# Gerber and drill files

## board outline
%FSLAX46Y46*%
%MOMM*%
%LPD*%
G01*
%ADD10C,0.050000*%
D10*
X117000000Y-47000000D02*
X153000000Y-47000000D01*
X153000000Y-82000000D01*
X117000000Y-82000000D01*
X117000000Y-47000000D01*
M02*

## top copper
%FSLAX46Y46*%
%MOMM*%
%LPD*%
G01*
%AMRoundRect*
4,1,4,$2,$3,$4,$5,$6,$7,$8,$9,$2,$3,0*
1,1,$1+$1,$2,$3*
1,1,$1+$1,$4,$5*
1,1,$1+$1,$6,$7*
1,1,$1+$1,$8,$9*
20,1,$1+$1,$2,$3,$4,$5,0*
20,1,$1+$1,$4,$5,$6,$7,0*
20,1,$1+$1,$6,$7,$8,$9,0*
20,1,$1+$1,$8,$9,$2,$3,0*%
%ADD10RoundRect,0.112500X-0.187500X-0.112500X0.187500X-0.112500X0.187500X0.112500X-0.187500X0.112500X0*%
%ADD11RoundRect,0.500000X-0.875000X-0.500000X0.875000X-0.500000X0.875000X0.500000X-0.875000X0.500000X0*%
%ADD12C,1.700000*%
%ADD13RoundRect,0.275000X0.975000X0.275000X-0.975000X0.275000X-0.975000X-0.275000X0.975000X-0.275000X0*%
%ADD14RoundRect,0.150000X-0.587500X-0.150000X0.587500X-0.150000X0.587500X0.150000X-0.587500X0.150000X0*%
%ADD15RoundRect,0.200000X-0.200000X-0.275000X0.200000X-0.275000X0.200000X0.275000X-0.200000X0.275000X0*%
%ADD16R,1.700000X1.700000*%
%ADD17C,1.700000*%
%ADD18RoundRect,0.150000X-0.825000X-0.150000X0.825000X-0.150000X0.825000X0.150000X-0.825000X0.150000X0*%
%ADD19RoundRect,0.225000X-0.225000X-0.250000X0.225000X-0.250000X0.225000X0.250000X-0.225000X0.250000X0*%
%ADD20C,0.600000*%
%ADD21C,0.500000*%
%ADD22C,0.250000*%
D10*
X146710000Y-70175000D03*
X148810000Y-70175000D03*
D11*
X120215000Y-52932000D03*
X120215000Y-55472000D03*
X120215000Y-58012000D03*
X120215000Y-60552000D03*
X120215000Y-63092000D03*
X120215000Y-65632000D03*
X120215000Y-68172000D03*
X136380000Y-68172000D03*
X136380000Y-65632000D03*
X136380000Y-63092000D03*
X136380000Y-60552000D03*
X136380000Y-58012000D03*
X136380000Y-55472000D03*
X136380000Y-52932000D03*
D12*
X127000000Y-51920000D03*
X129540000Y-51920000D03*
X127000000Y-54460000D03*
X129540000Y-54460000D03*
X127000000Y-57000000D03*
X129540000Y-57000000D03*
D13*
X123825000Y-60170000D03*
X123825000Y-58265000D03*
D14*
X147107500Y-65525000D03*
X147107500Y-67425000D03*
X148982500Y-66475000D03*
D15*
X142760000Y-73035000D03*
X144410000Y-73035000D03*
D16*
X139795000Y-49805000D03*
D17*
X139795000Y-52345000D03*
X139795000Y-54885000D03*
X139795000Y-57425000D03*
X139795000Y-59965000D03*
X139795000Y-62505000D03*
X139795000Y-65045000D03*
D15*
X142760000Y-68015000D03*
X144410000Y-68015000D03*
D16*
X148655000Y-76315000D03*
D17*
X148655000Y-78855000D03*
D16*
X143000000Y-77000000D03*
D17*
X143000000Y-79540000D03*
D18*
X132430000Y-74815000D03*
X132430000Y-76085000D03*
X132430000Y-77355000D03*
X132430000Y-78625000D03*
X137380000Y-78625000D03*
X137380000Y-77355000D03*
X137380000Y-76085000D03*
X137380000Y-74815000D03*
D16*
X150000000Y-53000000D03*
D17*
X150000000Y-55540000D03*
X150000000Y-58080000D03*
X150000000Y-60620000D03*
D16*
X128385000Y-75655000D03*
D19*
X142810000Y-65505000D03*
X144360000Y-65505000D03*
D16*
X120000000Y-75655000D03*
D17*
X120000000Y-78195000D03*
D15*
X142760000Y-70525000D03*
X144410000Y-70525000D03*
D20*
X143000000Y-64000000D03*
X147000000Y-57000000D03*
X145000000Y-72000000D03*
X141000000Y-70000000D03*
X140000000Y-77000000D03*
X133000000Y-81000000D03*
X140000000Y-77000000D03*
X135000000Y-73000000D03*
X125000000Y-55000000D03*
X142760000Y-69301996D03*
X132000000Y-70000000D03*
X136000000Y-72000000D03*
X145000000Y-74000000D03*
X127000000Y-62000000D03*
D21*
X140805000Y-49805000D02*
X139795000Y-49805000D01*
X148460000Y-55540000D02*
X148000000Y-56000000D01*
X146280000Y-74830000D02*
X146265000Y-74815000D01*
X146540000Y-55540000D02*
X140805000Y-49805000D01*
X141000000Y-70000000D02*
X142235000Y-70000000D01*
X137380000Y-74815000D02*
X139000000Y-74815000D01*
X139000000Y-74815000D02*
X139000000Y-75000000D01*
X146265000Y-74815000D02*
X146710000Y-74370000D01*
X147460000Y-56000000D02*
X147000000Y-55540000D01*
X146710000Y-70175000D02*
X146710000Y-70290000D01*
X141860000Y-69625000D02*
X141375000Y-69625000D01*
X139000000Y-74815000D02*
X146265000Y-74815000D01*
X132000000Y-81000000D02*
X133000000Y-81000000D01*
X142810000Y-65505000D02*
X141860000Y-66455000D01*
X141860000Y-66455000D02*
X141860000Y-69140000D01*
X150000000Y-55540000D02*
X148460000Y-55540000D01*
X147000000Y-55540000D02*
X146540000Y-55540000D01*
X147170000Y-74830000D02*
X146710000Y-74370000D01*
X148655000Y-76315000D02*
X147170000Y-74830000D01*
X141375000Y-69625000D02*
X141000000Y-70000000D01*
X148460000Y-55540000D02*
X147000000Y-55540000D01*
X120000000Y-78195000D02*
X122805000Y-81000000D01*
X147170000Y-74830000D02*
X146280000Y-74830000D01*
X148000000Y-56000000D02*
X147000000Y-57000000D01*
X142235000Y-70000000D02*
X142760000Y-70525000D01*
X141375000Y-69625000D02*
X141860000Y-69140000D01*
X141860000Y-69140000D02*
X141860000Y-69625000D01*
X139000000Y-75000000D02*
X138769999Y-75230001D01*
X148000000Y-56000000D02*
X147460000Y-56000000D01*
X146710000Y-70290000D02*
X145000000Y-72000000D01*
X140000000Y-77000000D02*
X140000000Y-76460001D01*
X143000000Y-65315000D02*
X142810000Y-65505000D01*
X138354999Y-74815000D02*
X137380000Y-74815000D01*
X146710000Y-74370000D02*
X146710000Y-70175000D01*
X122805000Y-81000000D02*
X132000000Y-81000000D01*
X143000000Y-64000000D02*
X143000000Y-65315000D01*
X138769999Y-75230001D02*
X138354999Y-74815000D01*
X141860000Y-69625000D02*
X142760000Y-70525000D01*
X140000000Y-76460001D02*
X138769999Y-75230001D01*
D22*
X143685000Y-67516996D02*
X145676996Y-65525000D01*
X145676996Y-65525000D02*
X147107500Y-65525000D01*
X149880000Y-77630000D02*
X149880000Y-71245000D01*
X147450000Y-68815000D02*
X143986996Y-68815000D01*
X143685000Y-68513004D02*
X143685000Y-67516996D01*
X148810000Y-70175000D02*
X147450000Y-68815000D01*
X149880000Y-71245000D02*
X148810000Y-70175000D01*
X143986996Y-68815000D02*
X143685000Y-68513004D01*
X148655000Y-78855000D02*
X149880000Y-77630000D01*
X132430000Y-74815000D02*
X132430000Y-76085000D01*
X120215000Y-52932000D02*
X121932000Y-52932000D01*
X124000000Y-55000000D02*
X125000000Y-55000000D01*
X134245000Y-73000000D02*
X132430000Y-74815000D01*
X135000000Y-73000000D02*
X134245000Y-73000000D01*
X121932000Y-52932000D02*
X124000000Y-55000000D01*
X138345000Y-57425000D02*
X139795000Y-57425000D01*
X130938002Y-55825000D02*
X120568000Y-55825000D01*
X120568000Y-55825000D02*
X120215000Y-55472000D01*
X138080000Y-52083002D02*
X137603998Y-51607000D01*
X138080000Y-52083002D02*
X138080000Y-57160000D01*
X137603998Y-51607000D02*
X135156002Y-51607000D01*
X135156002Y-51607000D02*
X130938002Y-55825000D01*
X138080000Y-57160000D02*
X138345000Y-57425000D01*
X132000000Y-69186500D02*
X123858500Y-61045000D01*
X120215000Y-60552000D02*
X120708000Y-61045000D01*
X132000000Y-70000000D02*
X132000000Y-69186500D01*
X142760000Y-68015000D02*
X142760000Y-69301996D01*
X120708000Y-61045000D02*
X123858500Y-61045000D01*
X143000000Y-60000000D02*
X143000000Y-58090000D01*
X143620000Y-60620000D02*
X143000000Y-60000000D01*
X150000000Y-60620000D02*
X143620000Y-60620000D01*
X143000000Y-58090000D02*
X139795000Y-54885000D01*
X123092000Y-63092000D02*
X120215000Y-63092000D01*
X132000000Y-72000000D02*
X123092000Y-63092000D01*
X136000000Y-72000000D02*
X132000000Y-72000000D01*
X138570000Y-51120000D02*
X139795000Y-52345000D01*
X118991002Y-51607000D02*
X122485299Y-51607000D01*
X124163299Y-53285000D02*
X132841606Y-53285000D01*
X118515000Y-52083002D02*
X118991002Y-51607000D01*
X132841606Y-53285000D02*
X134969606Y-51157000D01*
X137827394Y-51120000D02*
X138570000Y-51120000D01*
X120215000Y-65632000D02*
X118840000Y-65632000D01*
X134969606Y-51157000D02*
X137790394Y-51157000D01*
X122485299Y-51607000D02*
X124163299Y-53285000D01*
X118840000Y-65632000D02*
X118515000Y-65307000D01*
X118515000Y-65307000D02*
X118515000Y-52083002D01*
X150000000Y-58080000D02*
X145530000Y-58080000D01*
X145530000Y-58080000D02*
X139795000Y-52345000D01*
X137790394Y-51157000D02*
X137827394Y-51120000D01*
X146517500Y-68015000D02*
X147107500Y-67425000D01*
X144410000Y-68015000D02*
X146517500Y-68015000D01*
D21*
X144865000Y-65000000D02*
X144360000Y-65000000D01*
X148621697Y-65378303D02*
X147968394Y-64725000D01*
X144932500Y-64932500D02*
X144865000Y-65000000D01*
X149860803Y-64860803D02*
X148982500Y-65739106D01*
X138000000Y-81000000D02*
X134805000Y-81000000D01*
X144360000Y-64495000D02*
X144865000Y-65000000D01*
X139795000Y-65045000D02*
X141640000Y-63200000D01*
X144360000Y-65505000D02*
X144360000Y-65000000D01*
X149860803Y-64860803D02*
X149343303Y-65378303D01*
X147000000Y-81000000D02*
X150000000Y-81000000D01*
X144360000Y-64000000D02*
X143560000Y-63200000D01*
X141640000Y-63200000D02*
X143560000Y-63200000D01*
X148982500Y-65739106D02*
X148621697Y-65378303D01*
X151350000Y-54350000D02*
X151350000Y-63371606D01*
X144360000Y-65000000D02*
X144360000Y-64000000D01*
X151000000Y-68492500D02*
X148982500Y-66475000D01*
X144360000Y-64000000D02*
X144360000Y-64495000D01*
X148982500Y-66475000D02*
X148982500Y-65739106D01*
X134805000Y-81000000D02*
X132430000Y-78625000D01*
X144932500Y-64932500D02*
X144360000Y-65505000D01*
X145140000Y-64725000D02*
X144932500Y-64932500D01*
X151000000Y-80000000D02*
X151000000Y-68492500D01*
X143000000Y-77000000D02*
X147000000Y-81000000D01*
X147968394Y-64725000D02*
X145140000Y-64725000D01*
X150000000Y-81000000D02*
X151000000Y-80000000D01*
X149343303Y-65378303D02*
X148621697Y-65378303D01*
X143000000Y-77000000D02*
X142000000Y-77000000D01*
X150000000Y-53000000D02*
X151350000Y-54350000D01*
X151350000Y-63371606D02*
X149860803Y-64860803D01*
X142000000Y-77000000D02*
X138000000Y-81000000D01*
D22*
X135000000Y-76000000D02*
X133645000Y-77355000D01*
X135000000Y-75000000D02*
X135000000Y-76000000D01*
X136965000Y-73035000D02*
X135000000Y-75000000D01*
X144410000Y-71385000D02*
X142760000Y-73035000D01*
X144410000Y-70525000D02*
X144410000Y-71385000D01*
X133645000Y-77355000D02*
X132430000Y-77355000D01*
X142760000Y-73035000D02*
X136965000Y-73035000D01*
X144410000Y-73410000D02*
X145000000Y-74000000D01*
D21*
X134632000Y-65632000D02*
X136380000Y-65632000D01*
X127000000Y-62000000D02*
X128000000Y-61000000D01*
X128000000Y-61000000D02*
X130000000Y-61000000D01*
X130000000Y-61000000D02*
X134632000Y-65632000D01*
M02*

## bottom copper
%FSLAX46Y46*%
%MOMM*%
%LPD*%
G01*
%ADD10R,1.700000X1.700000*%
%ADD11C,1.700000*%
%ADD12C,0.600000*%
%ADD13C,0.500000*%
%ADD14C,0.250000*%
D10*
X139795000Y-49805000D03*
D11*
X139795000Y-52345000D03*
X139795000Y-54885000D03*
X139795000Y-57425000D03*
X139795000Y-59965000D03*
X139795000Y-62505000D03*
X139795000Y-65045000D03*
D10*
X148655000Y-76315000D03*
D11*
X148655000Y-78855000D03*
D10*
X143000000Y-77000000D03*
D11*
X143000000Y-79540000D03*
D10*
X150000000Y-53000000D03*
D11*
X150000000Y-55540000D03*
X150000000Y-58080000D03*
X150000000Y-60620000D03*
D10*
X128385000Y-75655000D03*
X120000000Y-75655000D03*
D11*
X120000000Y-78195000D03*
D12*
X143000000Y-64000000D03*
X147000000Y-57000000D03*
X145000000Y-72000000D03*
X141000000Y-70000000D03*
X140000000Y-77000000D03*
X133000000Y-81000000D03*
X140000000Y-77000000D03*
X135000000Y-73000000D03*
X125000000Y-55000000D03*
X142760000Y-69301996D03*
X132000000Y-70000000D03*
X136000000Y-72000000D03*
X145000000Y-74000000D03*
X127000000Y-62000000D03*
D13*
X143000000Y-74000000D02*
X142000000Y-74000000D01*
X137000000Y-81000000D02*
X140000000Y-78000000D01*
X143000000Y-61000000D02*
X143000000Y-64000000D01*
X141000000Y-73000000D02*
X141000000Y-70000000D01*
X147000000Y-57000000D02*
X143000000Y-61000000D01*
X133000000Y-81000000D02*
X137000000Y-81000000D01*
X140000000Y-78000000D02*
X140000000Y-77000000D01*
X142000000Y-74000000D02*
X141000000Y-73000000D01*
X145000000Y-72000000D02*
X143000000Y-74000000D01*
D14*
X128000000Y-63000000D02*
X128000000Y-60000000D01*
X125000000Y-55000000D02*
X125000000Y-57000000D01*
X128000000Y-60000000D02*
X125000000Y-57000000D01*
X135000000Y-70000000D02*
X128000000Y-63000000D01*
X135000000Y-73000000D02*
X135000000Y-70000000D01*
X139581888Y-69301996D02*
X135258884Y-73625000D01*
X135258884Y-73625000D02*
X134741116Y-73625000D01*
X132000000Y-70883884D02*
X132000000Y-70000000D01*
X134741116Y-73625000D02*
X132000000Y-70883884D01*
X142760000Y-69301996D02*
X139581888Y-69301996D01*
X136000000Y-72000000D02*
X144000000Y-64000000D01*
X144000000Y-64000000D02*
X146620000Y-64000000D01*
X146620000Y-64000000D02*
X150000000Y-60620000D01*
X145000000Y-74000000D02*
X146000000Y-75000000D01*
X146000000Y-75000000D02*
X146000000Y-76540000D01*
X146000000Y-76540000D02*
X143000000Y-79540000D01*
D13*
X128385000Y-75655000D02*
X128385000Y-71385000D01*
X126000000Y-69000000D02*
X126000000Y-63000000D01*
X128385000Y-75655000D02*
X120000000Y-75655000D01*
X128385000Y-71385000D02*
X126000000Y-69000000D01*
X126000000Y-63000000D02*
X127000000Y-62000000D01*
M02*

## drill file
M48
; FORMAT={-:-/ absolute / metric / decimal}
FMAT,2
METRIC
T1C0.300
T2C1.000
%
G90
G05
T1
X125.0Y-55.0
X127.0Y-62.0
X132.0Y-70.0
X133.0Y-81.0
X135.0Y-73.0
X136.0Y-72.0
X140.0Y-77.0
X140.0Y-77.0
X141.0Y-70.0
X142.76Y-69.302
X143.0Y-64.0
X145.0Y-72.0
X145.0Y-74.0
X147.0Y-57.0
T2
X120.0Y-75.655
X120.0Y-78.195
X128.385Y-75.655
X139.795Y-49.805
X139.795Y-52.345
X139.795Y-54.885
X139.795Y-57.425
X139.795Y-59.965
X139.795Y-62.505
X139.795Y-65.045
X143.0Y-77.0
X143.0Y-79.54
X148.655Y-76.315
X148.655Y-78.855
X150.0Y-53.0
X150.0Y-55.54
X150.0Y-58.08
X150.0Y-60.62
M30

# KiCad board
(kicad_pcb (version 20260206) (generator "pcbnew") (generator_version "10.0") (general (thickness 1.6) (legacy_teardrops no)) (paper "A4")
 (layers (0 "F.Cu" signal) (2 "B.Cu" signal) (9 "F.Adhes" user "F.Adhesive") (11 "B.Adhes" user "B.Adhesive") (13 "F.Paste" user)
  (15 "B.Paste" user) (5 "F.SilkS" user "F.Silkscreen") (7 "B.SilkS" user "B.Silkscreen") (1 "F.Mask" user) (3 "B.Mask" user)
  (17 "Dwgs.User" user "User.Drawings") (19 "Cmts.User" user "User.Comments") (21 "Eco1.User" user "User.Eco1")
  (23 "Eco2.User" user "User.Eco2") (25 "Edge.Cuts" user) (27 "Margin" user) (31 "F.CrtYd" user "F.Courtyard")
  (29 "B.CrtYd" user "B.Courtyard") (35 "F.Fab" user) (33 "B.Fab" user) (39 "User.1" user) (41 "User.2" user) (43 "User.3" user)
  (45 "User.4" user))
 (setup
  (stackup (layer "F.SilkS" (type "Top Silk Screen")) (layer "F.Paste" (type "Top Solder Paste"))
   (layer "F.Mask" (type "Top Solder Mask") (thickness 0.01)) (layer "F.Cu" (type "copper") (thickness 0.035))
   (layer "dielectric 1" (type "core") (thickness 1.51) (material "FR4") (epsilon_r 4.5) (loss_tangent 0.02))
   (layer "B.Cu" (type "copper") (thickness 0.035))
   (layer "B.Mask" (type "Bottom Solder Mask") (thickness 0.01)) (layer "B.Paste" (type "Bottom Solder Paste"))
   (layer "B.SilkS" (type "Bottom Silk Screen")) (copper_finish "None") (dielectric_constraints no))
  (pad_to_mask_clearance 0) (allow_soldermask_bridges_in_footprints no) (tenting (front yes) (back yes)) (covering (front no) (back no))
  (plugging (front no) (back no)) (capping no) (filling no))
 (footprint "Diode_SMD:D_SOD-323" (layer "F.Cu") (at 147.76 70.175)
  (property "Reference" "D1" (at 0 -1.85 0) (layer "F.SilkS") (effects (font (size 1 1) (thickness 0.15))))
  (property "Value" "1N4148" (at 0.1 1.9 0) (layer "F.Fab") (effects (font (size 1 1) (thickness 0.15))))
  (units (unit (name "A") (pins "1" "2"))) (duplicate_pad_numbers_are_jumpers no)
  (pad "1" smd roundrect (at -1.05 0) (size 0.6 0.45) (layers "F.Cu" "F.Mask" "F.Paste") (roundrect_rratio 0.25) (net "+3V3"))
  (pad "2" smd roundrect (at 1.05 0) (size 0.6 0.45) (layers "F.Cu" "F.Mask" "F.Paste") (roundrect_rratio 0.25) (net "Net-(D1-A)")))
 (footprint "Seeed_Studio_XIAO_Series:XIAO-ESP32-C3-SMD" (layer "F.Cu") (at 119.38 71.052)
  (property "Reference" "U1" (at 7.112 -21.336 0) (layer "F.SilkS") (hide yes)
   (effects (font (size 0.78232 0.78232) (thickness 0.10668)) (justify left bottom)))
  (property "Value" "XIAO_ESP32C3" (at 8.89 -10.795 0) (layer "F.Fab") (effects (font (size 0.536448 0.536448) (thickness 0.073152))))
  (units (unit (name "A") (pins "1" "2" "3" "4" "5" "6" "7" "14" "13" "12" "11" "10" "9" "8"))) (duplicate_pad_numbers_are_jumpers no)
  (pad "1" smd roundrect (at 0.835 -18.12) (size 2.75 2) (layers "F.Cu" "F.Mask" "F.Paste") (roundrect_rratio 0.25) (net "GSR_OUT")
   (solder_mask_margin 0.0508) (thermal_bridge_angle 45))
  (pad "2" smd roundrect (at 0.835 -15.58) (size 2.75 2) (layers "F.Cu" "F.Mask" "F.Paste") (roundrect_rratio 0.25) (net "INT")
   (solder_mask_margin 0.0508) (thermal_bridge_angle 45))
  (pad "3" smd roundrect (at 0.835 -13.04) (size 2.75 2) (layers "F.Cu" "F.Mask" "F.Paste") (roundrect_rratio 0.25)
   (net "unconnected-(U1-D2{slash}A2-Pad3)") (solder_mask_margin 0.0508) (thermal_bridge_angle 45))
  (pad "4" smd roundrect (at 0.835 -10.5) (size 2.75 2) (layers "F.Cu" "F.Mask" "F.Paste") (roundrect_rratio 0.25)
   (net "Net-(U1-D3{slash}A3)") (solder_mask_margin 0.0508) (thermal_bridge_angle 45))
  (pad "5" smd roundrect (at 0.835 -7.96) (size 2.75 2) (layers "F.Cu" "F.Mask" "F.Paste") (roundrect_rratio 0.25) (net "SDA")
   (solder_mask_margin 0.0508) (thermal_bridge_angle 45))
  (pad "6" smd roundrect (at 0.835 -5.42) (size 2.75 2) (layers "F.Cu" "F.Mask" "F.Paste") (roundrect_rratio 0.25) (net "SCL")
   (solder_mask_margin 0.0508) (thermal_bridge_angle 45))
  (pad "7" smd roundrect (at 0.835 -2.88) (size 2.75 2) (layers "F.Cu" "F.Mask" "F.Paste") (roundrect_rratio 0.25)
   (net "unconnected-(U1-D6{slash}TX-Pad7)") (solder_mask_margin 0.0508) (thermal_bridge_angle 45))
  (pad "8" smd roundrect (at 17 -2.88) (size 2.75 2) (layers "F.Cu" "F.Mask" "F.Paste") (roundrect_rratio 0.25)
   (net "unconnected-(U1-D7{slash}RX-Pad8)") (solder_mask_margin 0.0508) (thermal_bridge_angle 45))
  (pad "9" smd roundrect (at 17 -5.42) (size 2.75 2) (layers "F.Cu" "F.Mask" "F.Paste") (roundrect_rratio 0.25) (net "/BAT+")
   (solder_mask_margin 0.0508) (thermal_bridge_angle 45))
  (pad "10" smd roundrect (at 17 -7.96) (size 2.75 2) (layers "F.Cu" "F.Mask" "F.Paste") (roundrect_rratio 0.25) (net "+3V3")
   (solder_mask_margin 0.0508) (thermal_bridge_angle 45))
  (pad "11" smd roundrect (at 17 -10.5) (size 2.75 2) (layers "F.Cu" "F.Mask" "F.Paste") (roundrect_rratio 0.25)
   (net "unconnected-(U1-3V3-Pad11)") (solder_mask_margin 0.0508) (thermal_bridge_angle 45))
  (pad "12" smd roundrect (at 17 -13.04) (size 2.75 2) (layers "F.Cu" "F.Mask" "F.Paste") (roundrect_rratio 0.25)
   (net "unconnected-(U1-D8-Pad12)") (solder_mask_margin 0.0508) (thermal_bridge_angle 45))
  (pad "13" smd roundrect (at 17 -15.58) (size 2.75 2) (layers "F.Cu" "F.Mask" "F.Paste") (roundrect_rratio 0.25)
   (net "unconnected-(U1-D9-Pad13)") (solder_mask_margin 0.0508) (thermal_bridge_angle 45))
  (pad "14" smd roundrect (at 17 -18.12) (size 2.75 2) (layers "F.Cu" "F.Mask" "F.Paste") (roundrect_rratio 0.25)
   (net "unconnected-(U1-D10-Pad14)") (solder_mask_margin 0.0508) (thermal_bridge_angle 45))
  (pad "15" smd circle (at 7.62 -19.132) (size 1.7 1.7) (layers "F.Cu" "F.Mask" "F.Paste"))
  (pad "16" smd circle (at 10.16 -19.132) (size 1.7 1.7) (layers "F.Cu" "F.Mask" "F.Paste"))
  (pad "17" smd circle (at 7.62 -16.592) (size 1.7 1.7) (layers "F.Cu" "F.Mask" "F.Paste"))
  (pad "18" smd circle (at 10.16 -16.592) (size 1.7 1.7) (layers "F.Cu" "F.Mask" "F.Paste"))
  (pad "19" smd circle (at 7.62 -14.052) (size 1.7 1.7) (layers "F.Cu" "F.Mask" "F.Paste"))
  (pad "20" smd circle (at 10.16 -14.052) (size 1.7 1.7) (layers "F.Cu" "F.Mask" "F.Paste"))
  (pad "21" smd roundrect (at 4.445 -10.882 180) (size 2.5 1.1) (layers "F.Cu" "F.Mask" "F.Paste") (roundrect_rratio 0.25)
   (thermal_bridge_angle 45))
  (pad "22" smd roundrect (at 4.445 -12.787 180) (size 2.5 1.1) (layers "F.Cu" "F.Mask" "F.Paste") (roundrect_rratio 0.25)
   (thermal_bridge_angle 45)))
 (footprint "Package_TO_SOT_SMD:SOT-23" (layer "F.Cu") (at 148.045 66.475)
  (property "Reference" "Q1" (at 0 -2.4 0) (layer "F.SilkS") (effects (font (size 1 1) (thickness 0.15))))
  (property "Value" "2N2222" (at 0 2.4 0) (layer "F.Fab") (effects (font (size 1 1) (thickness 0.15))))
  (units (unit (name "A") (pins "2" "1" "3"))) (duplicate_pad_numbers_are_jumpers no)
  (pad "1" smd roundrect (at -0.9375 -0.95) (size 1.475 0.6) (layers "F.Cu" "F.Mask" "F.Paste") (roundrect_rratio 0.25) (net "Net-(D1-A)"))
  (pad "2" smd roundrect (at -0.9375 0.95) (size 1.475 0.6) (layers "F.Cu" "F.Mask" "F.Paste") (roundrect_rratio 0.25) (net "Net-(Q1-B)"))
  (pad "3" smd roundrect (at 0.9375 0) (size 1.475 0.6) (layers "F.Cu" "F.Mask" "F.Paste") (roundrect_rratio 0.25) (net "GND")))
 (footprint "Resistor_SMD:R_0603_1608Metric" (layer "F.Cu") (at 143.585 73.035)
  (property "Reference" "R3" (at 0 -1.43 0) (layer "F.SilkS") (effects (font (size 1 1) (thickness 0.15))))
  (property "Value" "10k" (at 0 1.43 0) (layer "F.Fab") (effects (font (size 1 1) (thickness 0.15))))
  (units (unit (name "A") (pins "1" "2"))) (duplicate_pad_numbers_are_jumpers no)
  (pad "1" smd roundrect (at -0.825 0) (size 0.8 0.95) (layers "F.Cu" "F.Mask" "F.Paste") (roundrect_rratio 0.25) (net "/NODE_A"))
  (pad "2" smd roundrect (at 0.825 0) (size 0.8 0.95) (layers "F.Cu" "F.Mask" "F.Paste") (roundrect_rratio 0.25) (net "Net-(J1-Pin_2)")))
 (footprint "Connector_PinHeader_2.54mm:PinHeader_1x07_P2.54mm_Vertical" (layer "F.Cu") (at 139.795 49.805)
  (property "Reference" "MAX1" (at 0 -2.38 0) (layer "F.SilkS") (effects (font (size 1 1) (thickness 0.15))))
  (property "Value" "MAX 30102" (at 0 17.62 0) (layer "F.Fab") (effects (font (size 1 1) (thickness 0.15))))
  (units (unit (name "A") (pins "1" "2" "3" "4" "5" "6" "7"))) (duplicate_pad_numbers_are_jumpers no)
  (pad "1" thru_hole rect (at 0 0) (size 1.7 1.7) (drill 1) (layers "*.Cu" "*.Mask") (remove_unused_layers no) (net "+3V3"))
  (pad "2" thru_hole circle (at 0 2.54) (size 1.7 1.7) (drill 1) (layers "*.Cu" "*.Mask") (remove_unused_layers no) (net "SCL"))
  (pad "3" thru_hole circle (at 0 5.08) (size 1.7 1.7) (drill 1) (layers "*.Cu" "*.Mask") (remove_unused_layers no) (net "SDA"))
  (pad "4" thru_hole circle (at 0 7.62) (size 1.7 1.7) (drill 1) (layers "*.Cu" "*.Mask") (remove_unused_layers no) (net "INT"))
  (pad "5" thru_hole circle (at 0 10.16) (size 1.7 1.7) (drill 1) (layers "*.Cu" "*.Mask") (remove_unused_layers no)
   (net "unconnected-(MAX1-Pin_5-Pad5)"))
  (pad "6" thru_hole circle (at 0 12.7) (size 1.7 1.7) (drill 1) (layers "*.Cu" "*.Mask") (remove_unused_layers no)
   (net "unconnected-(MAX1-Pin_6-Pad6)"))
  (pad "7" thru_hole circle (at 0 15.24) (size 1.7 1.7) (drill 1) (layers "*.Cu" "*.Mask") (remove_unused_layers no) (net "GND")))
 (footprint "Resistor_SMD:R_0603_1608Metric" (layer "F.Cu") (at 143.585 68.015)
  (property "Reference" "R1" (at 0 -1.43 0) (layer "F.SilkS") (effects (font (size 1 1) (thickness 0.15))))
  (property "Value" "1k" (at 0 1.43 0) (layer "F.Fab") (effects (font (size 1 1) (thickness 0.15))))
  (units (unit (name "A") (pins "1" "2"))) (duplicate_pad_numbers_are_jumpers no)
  (pad "1" smd roundrect (at -0.825 0) (size 0.8 0.95) (layers "F.Cu" "F.Mask" "F.Paste") (roundrect_rratio 0.25)
   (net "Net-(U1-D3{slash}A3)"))
  (pad "2" smd roundrect (at 0.825 0) (size 0.8 0.95) (layers "F.Cu" "F.Mask" "F.Paste") (roundrect_rratio 0.25) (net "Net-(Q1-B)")))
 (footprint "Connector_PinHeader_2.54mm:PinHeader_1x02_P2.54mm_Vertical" (layer "F.Cu") (at 148.655 76.315)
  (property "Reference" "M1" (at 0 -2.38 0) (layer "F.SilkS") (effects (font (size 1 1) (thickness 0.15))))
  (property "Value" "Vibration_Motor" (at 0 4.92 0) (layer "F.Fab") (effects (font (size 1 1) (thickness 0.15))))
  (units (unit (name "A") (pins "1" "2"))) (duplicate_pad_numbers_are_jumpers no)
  (pad "1" thru_hole rect (at 0 0) (size 1.7 1.7) (drill 1) (layers "*.Cu" "*.Mask") (remove_unused_layers no) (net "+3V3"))
  (pad "2" thru_hole circle (at 0 2.54) (size 1.7 1.7) (drill 1) (layers "*.Cu" "*.Mask") (remove_unused_layers no) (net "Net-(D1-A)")))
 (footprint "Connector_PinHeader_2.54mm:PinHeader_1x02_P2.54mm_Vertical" (layer "F.Cu") (at 143 77)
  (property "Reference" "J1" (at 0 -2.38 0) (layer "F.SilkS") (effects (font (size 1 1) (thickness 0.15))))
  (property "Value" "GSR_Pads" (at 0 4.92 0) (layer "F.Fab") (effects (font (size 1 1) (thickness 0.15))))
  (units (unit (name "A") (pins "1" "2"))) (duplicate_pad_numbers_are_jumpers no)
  (pad "1" thru_hole rect (at 0 0) (size 1.7 1.7) (drill 1) (layers "*.Cu" "*.Mask") (remove_unused_layers no) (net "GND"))
  (pad "2" thru_hole circle (at 0 2.54) (size 1.7 1.7) (drill 1) (layers "*.Cu" "*.Mask") (remove_unused_layers no) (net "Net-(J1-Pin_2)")))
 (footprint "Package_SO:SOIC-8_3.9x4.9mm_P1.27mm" (layer "F.Cu") (at 134.905 76.72)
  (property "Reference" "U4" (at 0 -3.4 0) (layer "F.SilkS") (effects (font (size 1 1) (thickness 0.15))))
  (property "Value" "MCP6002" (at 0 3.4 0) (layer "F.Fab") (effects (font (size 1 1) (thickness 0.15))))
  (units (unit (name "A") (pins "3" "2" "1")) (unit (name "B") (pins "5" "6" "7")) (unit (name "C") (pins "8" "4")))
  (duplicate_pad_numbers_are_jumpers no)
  (pad "1" smd roundrect (at -2.475 -1.905) (size 1.95 0.6) (layers "F.Cu" "F.Mask" "F.Paste") (roundrect_rratio 0.25) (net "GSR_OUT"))
  (pad "2" smd roundrect (at -2.475 -0.635) (size 1.95 0.6) (layers "F.Cu" "F.Mask" "F.Paste") (roundrect_rratio 0.25) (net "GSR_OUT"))
  (pad "3" smd roundrect (at -2.475 0.635) (size 1.95 0.6) (layers "F.Cu" "F.Mask" "F.Paste") (roundrect_rratio 0.25) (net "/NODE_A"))
  (pad "4" smd roundrect (at -2.475 1.905) (size 1.95 0.6) (layers "F.Cu" "F.Mask" "F.Paste") (roundrect_rratio 0.25) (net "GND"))
  (pad "5" smd roundrect (at 2.475 1.905) (size 1.95 0.6) (layers "F.Cu" "F.Mask" "F.Paste") (roundrect_rratio 0.25))
  (pad "6" smd roundrect (at 2.475 0.635) (size 1.95 0.6) (layers "F.Cu" "F.Mask" "F.Paste") (roundrect_rratio 0.25))
  (pad "7" smd roundrect (at 2.475 -0.635) (size 1.95 0.6) (layers "F.Cu" "F.Mask" "F.Paste") (roundrect_rratio 0.25))
  (pad "8" smd roundrect (at 2.475 -1.905) (size 1.95 0.6) (layers "F.Cu" "F.Mask" "F.Paste") (roundrect_rratio 0.25) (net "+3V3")))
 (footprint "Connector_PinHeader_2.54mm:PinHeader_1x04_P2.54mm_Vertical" (layer "F.Cu") (at 150 53)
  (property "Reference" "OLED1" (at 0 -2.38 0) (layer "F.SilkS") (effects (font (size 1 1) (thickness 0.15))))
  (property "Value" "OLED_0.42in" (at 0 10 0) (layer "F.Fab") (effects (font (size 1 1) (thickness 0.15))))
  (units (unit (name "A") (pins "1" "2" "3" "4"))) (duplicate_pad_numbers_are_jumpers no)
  (pad "1" thru_hole rect (at 0 0) (size 1.7 1.7) (drill 1) (layers "*.Cu" "*.Mask") (remove_unused_layers no) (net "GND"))
  (pad "2" thru_hole circle (at 0 2.54) (size 1.7 1.7) (drill 1) (layers "*.Cu" "*.Mask") (remove_unused_layers no) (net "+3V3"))
  (pad "3" thru_hole circle (at 0 5.08) (size 1.7 1.7) (drill 1) (layers "*.Cu" "*.Mask") (remove_unused_layers no) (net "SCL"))
  (pad "4" thru_hole circle (at 0 7.62) (size 1.7 1.7) (drill 1) (layers "*.Cu" "*.Mask") (remove_unused_layers no) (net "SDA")))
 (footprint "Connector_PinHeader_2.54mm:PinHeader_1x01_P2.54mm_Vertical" (layer "F.Cu") (at 128.385 75.655)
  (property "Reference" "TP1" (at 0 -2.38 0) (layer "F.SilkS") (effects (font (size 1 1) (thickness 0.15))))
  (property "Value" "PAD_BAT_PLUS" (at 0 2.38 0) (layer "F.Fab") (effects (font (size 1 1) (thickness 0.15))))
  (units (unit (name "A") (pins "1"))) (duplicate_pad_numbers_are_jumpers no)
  (pad "1" thru_hole rect (at 0 0) (size 1.7 1.7) (drill 1) (layers "*.Cu" "*.Mask") (remove_unused_layers no) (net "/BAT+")))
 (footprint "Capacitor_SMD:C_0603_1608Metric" (layer "F.Cu") (at 143.585 65.505)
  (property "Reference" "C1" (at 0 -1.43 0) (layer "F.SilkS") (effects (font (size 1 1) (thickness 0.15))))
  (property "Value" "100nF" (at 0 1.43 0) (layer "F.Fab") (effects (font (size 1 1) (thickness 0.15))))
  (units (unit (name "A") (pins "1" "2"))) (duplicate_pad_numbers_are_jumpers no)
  (pad "1" smd roundrect (at -0.775 0) (size 0.9 0.95) (layers "F.Cu" "F.Mask" "F.Paste") (roundrect_rratio 0.25) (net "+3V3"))
  (pad "2" smd roundrect (at 0.775 0) (size 0.9 0.95) (layers "F.Cu" "F.Mask" "F.Paste") (roundrect_rratio 0.25) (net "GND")))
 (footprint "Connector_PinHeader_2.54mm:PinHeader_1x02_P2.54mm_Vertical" (layer "F.Cu") (at 120 75.655)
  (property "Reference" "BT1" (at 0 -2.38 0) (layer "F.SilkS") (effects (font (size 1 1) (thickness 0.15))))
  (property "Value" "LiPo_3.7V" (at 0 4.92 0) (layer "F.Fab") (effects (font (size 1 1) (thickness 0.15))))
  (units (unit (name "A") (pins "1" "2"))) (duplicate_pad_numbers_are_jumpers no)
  (pad "1" thru_hole rect (at 0 0) (size 1.7 1.7) (drill 1) (layers "*.Cu" "*.Mask") (remove_unused_layers no) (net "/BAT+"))
  (pad "2" thru_hole circle (at 0 2.54) (size 1.7 1.7) (drill 1) (layers "*.Cu" "*.Mask") (remove_unused_layers no) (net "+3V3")))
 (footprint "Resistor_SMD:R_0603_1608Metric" (layer "F.Cu") (at 143.585 70.525)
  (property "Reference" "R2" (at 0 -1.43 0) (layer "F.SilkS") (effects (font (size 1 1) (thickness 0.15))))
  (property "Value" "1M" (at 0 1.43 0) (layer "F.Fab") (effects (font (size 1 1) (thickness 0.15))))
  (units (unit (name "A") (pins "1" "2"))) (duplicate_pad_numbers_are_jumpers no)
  (pad "1" smd roundrect (at -0.825 0) (size 0.8 0.95) (layers "F.Cu" "F.Mask" "F.Paste") (roundrect_rratio 0.25) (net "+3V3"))
  (pad "2" smd roundrect (at 0.825 0) (size 0.8 0.95) (layers "F.Cu" "F.Mask" "F.Paste") (roundrect_rratio 0.25) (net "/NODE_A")))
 (gr_rect (start 117 47) (end 153 82) (stroke (width 0.05) (type default)) (fill no) (layer "Edge.Cuts"))
 (segment (start 140.805 49.805) (end 139.795 49.805) (width 0.5) (layer "F.Cu") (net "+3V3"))
 (segment (start 148.46 55.54) (end 148 56) (width 0.5) (layer "F.Cu") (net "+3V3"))
 (segment (start 146.28 74.83) (end 146.265 74.815) (width 0.5) (layer "F.Cu") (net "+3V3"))
 (segment (start 146.54 55.54) (end 140.805 49.805) (width 0.5) (layer "F.Cu") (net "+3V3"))
 (segment (start 141 70) (end 142.235 70) (width 0.5) (layer "F.Cu") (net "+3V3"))
 (segment (start 137.38 74.815) (end 139 74.815) (width 0.5) (layer "F.Cu") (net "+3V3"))
 (segment (start 139 74.815) (end 139 75) (width 0.5) (layer "F.Cu") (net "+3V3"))
 (segment (start 146.265 74.815) (end 146.71 74.37) (width 0.5) (layer "F.Cu") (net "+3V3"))
 (segment (start 147.46 56) (end 147 55.54) (width 0.5) (layer "F.Cu") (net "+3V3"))
 (segment (start 146.71 70.175) (end 146.71 70.29) (width 0.5) (layer "F.Cu") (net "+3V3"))
 (segment (start 141.86 69.625) (end 141.375 69.625) (width 0.5) (layer "F.Cu") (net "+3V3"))
 (segment (start 139 74.815) (end 146.265 74.815) (width 0.5) (layer "F.Cu") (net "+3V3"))
 (segment (start 132 81) (end 133 81) (width 0.5) (layer "F.Cu") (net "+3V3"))
 (segment (start 142.81 65.505) (end 141.86 66.455) (width 0.5) (layer "F.Cu") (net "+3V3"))
 (segment (start 141.86 66.455) (end 141.86 69.14) (width 0.5) (layer "F.Cu") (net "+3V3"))
 (segment (start 150 55.54) (end 148.46 55.54) (width 0.5) (layer "F.Cu") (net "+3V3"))
 (segment (start 147 55.54) (end 146.54 55.54) (width 0.5) (layer "F.Cu") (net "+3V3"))
 (segment (start 147.17 74.83) (end 146.71 74.37) (width 0.5) (layer "F.Cu") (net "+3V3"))
 (segment (start 148.655 76.315) (end 147.17 74.83) (width 0.5) (layer "F.Cu") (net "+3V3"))
 (segment (start 141.375 69.625) (end 141 70) (width 0.5) (layer "F.Cu") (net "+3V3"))
 (segment (start 148.46 55.54) (end 147 55.54) (width 0.5) (layer "F.Cu") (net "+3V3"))
 (segment (start 120 78.195) (end 122.805 81) (width 0.5) (layer "F.Cu") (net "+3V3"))
 (segment (start 147.17 74.83) (end 146.28 74.83) (width 0.5) (layer "F.Cu") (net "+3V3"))
 (segment (start 148 56) (end 147 57) (width 0.5) (layer "F.Cu") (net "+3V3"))
 (segment (start 142.235 70) (end 142.76 70.525) (width 0.5) (layer "F.Cu") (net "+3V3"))
 (segment (start 141.375 69.625) (end 141.86 69.14) (width 0.5) (layer "F.Cu") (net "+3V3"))
 (segment (start 141.86 69.14) (end 141.86 69.625) (width 0.5) (layer "F.Cu") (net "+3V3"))
 (segment (start 139 75) (end 138.769999 75.230001) (width 0.5) (layer "F.Cu") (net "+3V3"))
 (segment (start 148 56) (end 147.46 56) (width 0.5) (layer "F.Cu") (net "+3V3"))
 (segment (start 146.71 70.29) (end 145 72) (width 0.5) (layer "F.Cu") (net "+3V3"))
 (segment (start 140 77) (end 140 76.460001) (width 0.5) (layer "F.Cu") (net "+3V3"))
 (segment (start 143 65.315) (end 142.81 65.505) (width 0.5) (layer "F.Cu") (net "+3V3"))
 (segment (start 138.354999 74.815) (end 137.38 74.815) (width 0.5) (layer "F.Cu") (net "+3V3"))
 (segment (start 146.71 74.37) (end 146.71 70.175) (width 0.5) (layer "F.Cu") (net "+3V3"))
 (segment (start 122.805 81) (end 132 81) (width 0.5) (layer "F.Cu") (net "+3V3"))
 (segment (start 143 64) (end 143 65.315) (width 0.5) (layer "F.Cu") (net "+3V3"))
 (segment (start 138.769999 75.230001) (end 138.354999 74.815) (width 0.5) (layer "F.Cu") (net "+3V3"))
 (segment (start 141.86 69.625) (end 142.76 70.525) (width 0.5) (layer "F.Cu") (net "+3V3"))
 (segment (start 140 76.460001) (end 138.769999 75.230001) (width 0.5) (layer "F.Cu") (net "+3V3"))
 (via (at 143 64) (size 0.6) (drill 0.3) (layers "F.Cu" "B.Cu") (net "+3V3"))
 (via (at 147 57) (size 0.6) (drill 0.3) (layers "F.Cu" "B.Cu") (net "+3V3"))
 (via (at 145 72) (size 0.6) (drill 0.3) (layers "F.Cu" "B.Cu") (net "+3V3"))
 (via (at 141 70) (size 0.6) (drill 0.3) (layers "F.Cu" "B.Cu") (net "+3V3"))
 (via (at 140 77) (size 0.6) (drill 0.3) (layers "F.Cu" "B.Cu") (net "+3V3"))
 (via (at 133 81) (size 0.6) (drill 0.3) (layers "F.Cu" "B.Cu") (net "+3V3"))
 (via (at 140 77) (size 0.6) (drill 0.3) (layers "F.Cu" "B.Cu") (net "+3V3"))
 (segment (start 143 74) (end 142 74) (width 0.5) (layer "B.Cu") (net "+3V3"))
 (segment (start 137 81) (end 140 78) (width 0.5) (layer "B.Cu") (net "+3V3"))
 (segment (start 143 61) (end 143 64) (width 0.5) (layer "B.Cu") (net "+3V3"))
 (segment (start 141 73) (end 141 70) (width 0.5) (layer "B.Cu") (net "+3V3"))
 (segment (start 147 57) (end 143 61) (width 0.5) (layer "B.Cu") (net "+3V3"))
 (segment (start 133 81) (end 137 81) (width 0.5) (layer "B.Cu") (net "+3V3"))
 (segment (start 140 78) (end 140 77) (width 0.5) (layer "B.Cu") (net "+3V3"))
 (segment (start 142 74) (end 141 73) (width 0.5) (layer "B.Cu") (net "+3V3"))
 (segment (start 145 72) (end 143 74) (width 0.5) (layer "B.Cu") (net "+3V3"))
 (segment (start 143.685 67.516996) (end 145.676996 65.525) (width 0.25) (layer "F.Cu") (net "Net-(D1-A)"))
 (segment (start 145.676996 65.525) (end 147.1075 65.525) (width 0.25) (layer "F.Cu") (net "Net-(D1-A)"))
 (segment (start 149.88 77.63) (end 149.88 71.245) (width 0.25) (layer "F.Cu") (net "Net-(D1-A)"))
 (segment (start 147.45 68.815) (end 143.986996 68.815) (width 0.25) (layer "F.Cu") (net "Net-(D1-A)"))
 (segment (start 143.685 68.513004) (end 143.685 67.516996) (width 0.25) (layer "F.Cu") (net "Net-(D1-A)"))
 (segment (start 148.81 70.175) (end 147.45 68.815) (width 0.25) (layer "F.Cu") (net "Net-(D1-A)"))
 (segment (start 149.88 71.245) (end 148.81 70.175) (width 0.25) (layer "F.Cu") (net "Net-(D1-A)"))
 (segment (start 143.986996 68.815) (end 143.685 68.513004) (width 0.25) (layer "F.Cu") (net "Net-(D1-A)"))
 (segment (start 148.655 78.855) (end 149.88 77.63) (width 0.25) (layer "F.Cu") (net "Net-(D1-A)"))
 (segment (start 132.43 74.815) (end 132.43 76.085) (width 0.25) (layer "F.Cu") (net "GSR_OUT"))
 (segment (start 120.215 52.932) (end 121.932 52.932) (width 0.25) (layer "F.Cu") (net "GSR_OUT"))
 (segment (start 124 55) (end 125 55) (width 0.25) (layer "F.Cu") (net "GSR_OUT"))
 (segment (start 134.245 73) (end 132.43 74.815) (width 0.25) (layer "F.Cu") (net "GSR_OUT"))
 (segment (start 135 73) (end 134.245 73) (width 0.25) (layer "F.Cu") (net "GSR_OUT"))
 (segment (start 121.932 52.932) (end 124 55) (width 0.25) (layer "F.Cu") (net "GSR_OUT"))
 (via (at 135 73) (size 0.6) (drill 0.3) (layers "F.Cu" "B.Cu") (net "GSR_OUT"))
 (via (at 125 55) (size 0.6) (drill 0.3) (layers "F.Cu" "B.Cu") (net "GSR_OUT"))
 (segment (start 128 63) (end 128 60) (width 0.25) (layer "B.Cu") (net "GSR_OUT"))
 (segment (start 125 55) (end 125 57) (width 0.25) (layer "B.Cu") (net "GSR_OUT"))
 (segment (start 128 60) (end 125 57) (width 0.25) (layer "B.Cu") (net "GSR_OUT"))
 (segment (start 135 70) (end 128 63) (width 0.25) (layer "B.Cu") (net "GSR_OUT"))
 (segment (start 135 73) (end 135 70) (width 0.25) (layer "B.Cu") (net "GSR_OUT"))
 (segment (start 138.345 57.425) (end 139.795 57.425) (width 0.25) (layer "F.Cu") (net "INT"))
 (segment (start 130.938002 55.825) (end 120.568 55.825) (width 0.25) (layer "F.Cu") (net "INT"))
 (segment (start 120.568 55.825) (end 120.215 55.472) (width 0.25) (layer "F.Cu") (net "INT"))
 (segment (start 138.08 52.083002) (end 137.603998 51.607) (width 0.25) (layer "F.Cu") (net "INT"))
 (segment (start 138.08 52.083002) (end 138.08 57.16) (width 0.25) (layer "F.Cu") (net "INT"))
 (segment (start 137.603998 51.607) (end 135.156002 51.607) (width 0.25) (layer "F.Cu") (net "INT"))
 (segment (start 135.156002 51.607) (end 130.938002 55.825) (width 0.25) (layer "F.Cu") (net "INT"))
 (segment (start 138.08 57.16) (end 138.345 57.425) (width 0.25) (layer "F.Cu") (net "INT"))
 (segment (start 132 69.1865) (end 123.8585 61.045) (width 0.25) (layer "F.Cu") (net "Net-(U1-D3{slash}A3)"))
 (segment (start 120.215 60.552) (end 120.708 61.045) (width 0.25) (layer "F.Cu") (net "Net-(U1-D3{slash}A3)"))
 (segment (start 132 70) (end 132 69.1865) (width 0.25) (layer "F.Cu") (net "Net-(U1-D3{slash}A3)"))
 (segment (start 142.76 68.015) (end 142.76 69.301996) (width 0.25) (layer "F.Cu") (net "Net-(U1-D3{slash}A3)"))
 (segment (start 120.708 61.045) (end 123.8585 61.045) (width 0.25) (layer "F.Cu") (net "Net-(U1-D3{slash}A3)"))
 (via (at 142.76 69.301996) (size 0.6) (drill 0.3) (layers "F.Cu" "B.Cu") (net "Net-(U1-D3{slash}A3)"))
 (via (at 132 70) (size 0.6) (drill 0.3) (layers "F.Cu" "B.Cu") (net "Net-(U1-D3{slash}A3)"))
 (segment (start 139.581888 69.301996) (end 135.258884 73.625) (width 0.25) (layer "B.Cu") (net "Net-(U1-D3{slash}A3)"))
 (segment (start 135.258884 73.625) (end 134.741116 73.625) (width 0.25) (layer "B.Cu") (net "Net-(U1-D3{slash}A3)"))
 (segment (start 132 70.883884) (end 132 70) (width 0.25) (layer "B.Cu") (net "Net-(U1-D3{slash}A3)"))
 (segment (start 134.741116 73.625) (end 132 70.883884) (width 0.25) (layer "B.Cu") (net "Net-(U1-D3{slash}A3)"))
 (segment (start 142.76 69.301996) (end 139.581888 69.301996) (width 0.25) (layer "B.Cu") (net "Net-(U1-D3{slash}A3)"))
 (segment (start 143 60) (end 143 58.09) (width 0.25) (layer "F.Cu") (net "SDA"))
 (segment (start 143.62 60.62) (end 143 60) (width 0.25) (layer "F.Cu") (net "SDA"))
 (segment (start 150 60.62) (end 143.62 60.62) (width 0.25) (layer "F.Cu") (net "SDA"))
 (segment (start 143 58.09) (end 139.795 54.885) (width 0.25) (layer "F.Cu") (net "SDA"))
 (segment (start 123.092 63.092) (end 120.215 63.092) (width 0.25) (layer "F.Cu") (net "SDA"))
 (segment (start 132 72) (end 123.092 63.092) (width 0.25) (layer "F.Cu") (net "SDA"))
 (segment (start 136 72) (end 132 72) (width 0.25) (layer "F.Cu") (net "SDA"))
 (via (at 136 72) (size 0.6) (drill 0.3) (layers "F.Cu" "B.Cu") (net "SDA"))
 (segment (start 136 72) (end 144 64) (width 0.25) (layer "B.Cu") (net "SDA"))
 (segment (start 144 64) (end 146.62 64) (width 0.25) (layer "B.Cu") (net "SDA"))
 (segment (start 146.62 64) (end 150 60.62) (width 0.25) (layer "B.Cu") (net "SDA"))
 (segment (start 138.57 51.12) (end 139.795 52.345) (width 0.25) (layer "F.Cu") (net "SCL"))
 (segment (start 118.991002 51.607) (end 122.485299 51.607) (width 0.25) (layer "F.Cu") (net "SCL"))
 (segment (start 124.163299 53.285) (end 132.841606 53.285) (width 0.25) (layer "F.Cu") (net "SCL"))
 (segment (start 118.515 52.083002) (end 118.991002 51.607) (width 0.25) (layer "F.Cu") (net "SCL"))
 (segment (start 132.841606 53.285) (end 134.969606 51.157) (width 0.25) (layer "F.Cu") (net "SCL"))
 (segment (start 137.827394 51.12) (end 138.57 51.12) (width 0.25) (layer "F.Cu") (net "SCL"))
 (segment (start 120.215 65.632) (end 118.84 65.632) (width 0.25) (layer "F.Cu") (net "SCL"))
 (segment (start 134.969606 51.157) (end 137.790394 51.157) (width 0.25) (layer "F.Cu") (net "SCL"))
 (segment (start 122.485299 51.607) (end 124.163299 53.285) (width 0.25) (layer "F.Cu") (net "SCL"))
 (segment (start 118.84 65.632) (end 118.515 65.307) (width 0.25) (layer "F.Cu") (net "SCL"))
 (segment (start 118.515 65.307) (end 118.515 52.083002) (width 0.25) (layer "F.Cu") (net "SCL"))
 (segment (start 150 58.08) (end 145.53 58.08) (width 0.25) (layer "F.Cu") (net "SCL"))
 (segment (start 145.53 58.08) (end 139.795 52.345) (width 0.25) (layer "F.Cu") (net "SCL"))
 (segment (start 137.790394 51.157) (end 137.827394 51.12) (width 0.25) (layer "F.Cu") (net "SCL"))
 (segment (start 146.5175 68.015) (end 147.1075 67.425) (width 0.25) (layer "F.Cu") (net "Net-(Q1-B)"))
 (segment (start 144.41 68.015) (end 146.5175 68.015) (width 0.25) (layer "F.Cu") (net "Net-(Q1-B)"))
 (segment (start 144.865 65) (end 144.36 65) (width 0.5) (layer "F.Cu") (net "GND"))
 (segment (start 148.621697 65.378303) (end 147.968394 64.725) (width 0.5) (layer "F.Cu") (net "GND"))
 (segment (start 144.9325 64.9325) (end 144.865 65) (width 0.5) (layer "F.Cu") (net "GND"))
 (segment (start 149.860803 64.860803) (end 148.9825 65.739106) (width 0.5) (layer "F.Cu") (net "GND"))
 (segment (start 138 81) (end 134.805 81) (width 0.5) (layer "F.Cu") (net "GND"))
 (segment (start 144.36 64.495) (end 144.865 65) (width 0.5) (layer "F.Cu") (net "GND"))
 (segment (start 139.795 65.045) (end 141.64 63.2) (width 0.5) (layer "F.Cu") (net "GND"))
 (segment (start 144.36 65.505) (end 144.36 65) (width 0.5) (layer "F.Cu") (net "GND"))
 (segment (start 149.860803 64.860803) (end 149.343303 65.378303) (width 0.5) (layer "F.Cu") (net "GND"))
 (segment (start 147 81) (end 150 81) (width 0.5) (layer "F.Cu") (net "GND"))
 (segment (start 144.36 64) (end 143.56 63.2) (width 0.5) (layer "F.Cu") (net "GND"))
 (segment (start 141.64 63.2) (end 143.56 63.2) (width 0.5) (layer "F.Cu") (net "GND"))
 (segment (start 148.9825 65.739106) (end 148.621697 65.378303) (width 0.5) (layer "F.Cu") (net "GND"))
 (segment (start 151.35 54.35) (end 151.35 63.371606) (width 0.5) (layer "F.Cu") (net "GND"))
 (segment (start 144.36 65) (end 144.36 64) (width 0.5) (layer "F.Cu") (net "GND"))
 (segment (start 151 68.4925) (end 148.9825 66.475) (width 0.5) (layer "F.Cu") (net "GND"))
 (segment (start 144.36 64) (end 144.36 64.495) (width 0.5) (layer "F.Cu") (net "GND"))
 (segment (start 148.9825 66.475) (end 148.9825 65.739106) (width 0.5) (layer "F.Cu") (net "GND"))
 (segment (start 134.805 81) (end 132.43 78.625) (width 0.5) (layer "F.Cu") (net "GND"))
 (segment (start 144.9325 64.9325) (end 144.36 65.505) (width 0.5) (layer "F.Cu") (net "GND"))
 (segment (start 145.14 64.725) (end 144.9325 64.9325) (width 0.5) (layer "F.Cu") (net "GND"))
 (segment (start 151 80) (end 151 68.4925) (width 0.5) (layer "F.Cu") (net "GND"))
 (segment (start 143 77) (end 147 81) (width 0.5) (layer "F.Cu") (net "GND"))
 (segment (start 147.968394 64.725) (end 145.14 64.725) (width 0.5) (layer "F.Cu") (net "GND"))
 (segment (start 150 81) (end 151 80) (width 0.5) (layer "F.Cu") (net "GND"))
 (segment (start 149.343303 65.378303) (end 148.621697 65.378303) (width 0.5) (layer "F.Cu") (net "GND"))
 (segment (start 143 77) (end 142 77) (width 0.5) (layer "F.Cu") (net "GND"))
 (segment (start 150 53) (end 151.35 54.35) (width 0.5) (layer "F.Cu") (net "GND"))
 (segment (start 151.35 63.371606) (end 149.860803 64.860803) (width 0.5) (layer "F.Cu") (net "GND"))
 (segment (start 142 77) (end 138 81) (width 0.5) (layer "F.Cu") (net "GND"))
 (segment (start 135 76) (end 133.645 77.355) (width 0.25) (layer "F.Cu") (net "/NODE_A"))
 (segment (start 135 75) (end 135 76) (width 0.25) (layer "F.Cu") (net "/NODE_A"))
 (segment (start 136.965 73.035) (end 135 75) (width 0.25) (layer "F.Cu") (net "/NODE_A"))
 (segment (start 144.41 71.385) (end 142.76 73.035) (width 0.25) (layer "F.Cu") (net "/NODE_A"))
 (segment (start 144.41 70.525) (end 144.41 71.385) (width 0.25) (layer "F.Cu") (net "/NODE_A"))
 (segment (start 133.645 77.355) (end 132.43 77.355) (width 0.25) (layer "F.Cu") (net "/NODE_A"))
 (segment (start 142.76 73.035) (end 136.965 73.035) (width 0.25) (layer "F.Cu") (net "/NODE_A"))
 (segment (start 144.41 73.41) (end 145 74) (width 0.25) (layer "F.Cu") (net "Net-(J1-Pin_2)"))
 (via (at 145 74) (size 0.6) (drill 0.3) (layers "F.Cu" "B.Cu") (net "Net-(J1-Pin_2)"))
 (segment (start 145 74) (end 146 75) (width 0.25) (layer "B.Cu") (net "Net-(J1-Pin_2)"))
 (segment (start 146 75) (end 146 76.54) (width 0.25) (layer "B.Cu") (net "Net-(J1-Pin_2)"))
 (segment (start 146 76.54) (end 143 79.54) (width 0.25) (layer "B.Cu") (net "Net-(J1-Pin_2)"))
 (segment (start 134.632 65.632) (end 136.38 65.632) (width 0.5) (layer "F.Cu") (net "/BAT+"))
 (segment (start 127 62) (end 128 61) (width 0.5) (layer "F.Cu") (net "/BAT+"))
 (segment (start 128 61) (end 130 61) (width 0.5) (layer "F.Cu") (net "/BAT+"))
 (segment (start 130 61) (end 134.632 65.632) (width 0.5) (layer "F.Cu") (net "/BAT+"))
 (via (at 127 62) (size 0.6) (drill 0.3) (layers "F.Cu" "B.Cu") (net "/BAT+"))
 (segment (start 128.385 75.655) (end 128.385 71.385) (width 0.5) (layer "B.Cu") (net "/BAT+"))
 (segment (start 126 69) (end 126 63) (width 0.5) (layer "B.Cu") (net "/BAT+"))
 (segment (start 128.385 75.655) (end 120 75.655) (width 0.5) (layer "B.Cu") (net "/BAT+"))
 (segment (start 128.385 71.385) (end 126 69) (width 0.5) (layer "B.Cu") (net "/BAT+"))
 (segment (start 126 63) (end 127 62) (width 0.5) (layer "B.Cu") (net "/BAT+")))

